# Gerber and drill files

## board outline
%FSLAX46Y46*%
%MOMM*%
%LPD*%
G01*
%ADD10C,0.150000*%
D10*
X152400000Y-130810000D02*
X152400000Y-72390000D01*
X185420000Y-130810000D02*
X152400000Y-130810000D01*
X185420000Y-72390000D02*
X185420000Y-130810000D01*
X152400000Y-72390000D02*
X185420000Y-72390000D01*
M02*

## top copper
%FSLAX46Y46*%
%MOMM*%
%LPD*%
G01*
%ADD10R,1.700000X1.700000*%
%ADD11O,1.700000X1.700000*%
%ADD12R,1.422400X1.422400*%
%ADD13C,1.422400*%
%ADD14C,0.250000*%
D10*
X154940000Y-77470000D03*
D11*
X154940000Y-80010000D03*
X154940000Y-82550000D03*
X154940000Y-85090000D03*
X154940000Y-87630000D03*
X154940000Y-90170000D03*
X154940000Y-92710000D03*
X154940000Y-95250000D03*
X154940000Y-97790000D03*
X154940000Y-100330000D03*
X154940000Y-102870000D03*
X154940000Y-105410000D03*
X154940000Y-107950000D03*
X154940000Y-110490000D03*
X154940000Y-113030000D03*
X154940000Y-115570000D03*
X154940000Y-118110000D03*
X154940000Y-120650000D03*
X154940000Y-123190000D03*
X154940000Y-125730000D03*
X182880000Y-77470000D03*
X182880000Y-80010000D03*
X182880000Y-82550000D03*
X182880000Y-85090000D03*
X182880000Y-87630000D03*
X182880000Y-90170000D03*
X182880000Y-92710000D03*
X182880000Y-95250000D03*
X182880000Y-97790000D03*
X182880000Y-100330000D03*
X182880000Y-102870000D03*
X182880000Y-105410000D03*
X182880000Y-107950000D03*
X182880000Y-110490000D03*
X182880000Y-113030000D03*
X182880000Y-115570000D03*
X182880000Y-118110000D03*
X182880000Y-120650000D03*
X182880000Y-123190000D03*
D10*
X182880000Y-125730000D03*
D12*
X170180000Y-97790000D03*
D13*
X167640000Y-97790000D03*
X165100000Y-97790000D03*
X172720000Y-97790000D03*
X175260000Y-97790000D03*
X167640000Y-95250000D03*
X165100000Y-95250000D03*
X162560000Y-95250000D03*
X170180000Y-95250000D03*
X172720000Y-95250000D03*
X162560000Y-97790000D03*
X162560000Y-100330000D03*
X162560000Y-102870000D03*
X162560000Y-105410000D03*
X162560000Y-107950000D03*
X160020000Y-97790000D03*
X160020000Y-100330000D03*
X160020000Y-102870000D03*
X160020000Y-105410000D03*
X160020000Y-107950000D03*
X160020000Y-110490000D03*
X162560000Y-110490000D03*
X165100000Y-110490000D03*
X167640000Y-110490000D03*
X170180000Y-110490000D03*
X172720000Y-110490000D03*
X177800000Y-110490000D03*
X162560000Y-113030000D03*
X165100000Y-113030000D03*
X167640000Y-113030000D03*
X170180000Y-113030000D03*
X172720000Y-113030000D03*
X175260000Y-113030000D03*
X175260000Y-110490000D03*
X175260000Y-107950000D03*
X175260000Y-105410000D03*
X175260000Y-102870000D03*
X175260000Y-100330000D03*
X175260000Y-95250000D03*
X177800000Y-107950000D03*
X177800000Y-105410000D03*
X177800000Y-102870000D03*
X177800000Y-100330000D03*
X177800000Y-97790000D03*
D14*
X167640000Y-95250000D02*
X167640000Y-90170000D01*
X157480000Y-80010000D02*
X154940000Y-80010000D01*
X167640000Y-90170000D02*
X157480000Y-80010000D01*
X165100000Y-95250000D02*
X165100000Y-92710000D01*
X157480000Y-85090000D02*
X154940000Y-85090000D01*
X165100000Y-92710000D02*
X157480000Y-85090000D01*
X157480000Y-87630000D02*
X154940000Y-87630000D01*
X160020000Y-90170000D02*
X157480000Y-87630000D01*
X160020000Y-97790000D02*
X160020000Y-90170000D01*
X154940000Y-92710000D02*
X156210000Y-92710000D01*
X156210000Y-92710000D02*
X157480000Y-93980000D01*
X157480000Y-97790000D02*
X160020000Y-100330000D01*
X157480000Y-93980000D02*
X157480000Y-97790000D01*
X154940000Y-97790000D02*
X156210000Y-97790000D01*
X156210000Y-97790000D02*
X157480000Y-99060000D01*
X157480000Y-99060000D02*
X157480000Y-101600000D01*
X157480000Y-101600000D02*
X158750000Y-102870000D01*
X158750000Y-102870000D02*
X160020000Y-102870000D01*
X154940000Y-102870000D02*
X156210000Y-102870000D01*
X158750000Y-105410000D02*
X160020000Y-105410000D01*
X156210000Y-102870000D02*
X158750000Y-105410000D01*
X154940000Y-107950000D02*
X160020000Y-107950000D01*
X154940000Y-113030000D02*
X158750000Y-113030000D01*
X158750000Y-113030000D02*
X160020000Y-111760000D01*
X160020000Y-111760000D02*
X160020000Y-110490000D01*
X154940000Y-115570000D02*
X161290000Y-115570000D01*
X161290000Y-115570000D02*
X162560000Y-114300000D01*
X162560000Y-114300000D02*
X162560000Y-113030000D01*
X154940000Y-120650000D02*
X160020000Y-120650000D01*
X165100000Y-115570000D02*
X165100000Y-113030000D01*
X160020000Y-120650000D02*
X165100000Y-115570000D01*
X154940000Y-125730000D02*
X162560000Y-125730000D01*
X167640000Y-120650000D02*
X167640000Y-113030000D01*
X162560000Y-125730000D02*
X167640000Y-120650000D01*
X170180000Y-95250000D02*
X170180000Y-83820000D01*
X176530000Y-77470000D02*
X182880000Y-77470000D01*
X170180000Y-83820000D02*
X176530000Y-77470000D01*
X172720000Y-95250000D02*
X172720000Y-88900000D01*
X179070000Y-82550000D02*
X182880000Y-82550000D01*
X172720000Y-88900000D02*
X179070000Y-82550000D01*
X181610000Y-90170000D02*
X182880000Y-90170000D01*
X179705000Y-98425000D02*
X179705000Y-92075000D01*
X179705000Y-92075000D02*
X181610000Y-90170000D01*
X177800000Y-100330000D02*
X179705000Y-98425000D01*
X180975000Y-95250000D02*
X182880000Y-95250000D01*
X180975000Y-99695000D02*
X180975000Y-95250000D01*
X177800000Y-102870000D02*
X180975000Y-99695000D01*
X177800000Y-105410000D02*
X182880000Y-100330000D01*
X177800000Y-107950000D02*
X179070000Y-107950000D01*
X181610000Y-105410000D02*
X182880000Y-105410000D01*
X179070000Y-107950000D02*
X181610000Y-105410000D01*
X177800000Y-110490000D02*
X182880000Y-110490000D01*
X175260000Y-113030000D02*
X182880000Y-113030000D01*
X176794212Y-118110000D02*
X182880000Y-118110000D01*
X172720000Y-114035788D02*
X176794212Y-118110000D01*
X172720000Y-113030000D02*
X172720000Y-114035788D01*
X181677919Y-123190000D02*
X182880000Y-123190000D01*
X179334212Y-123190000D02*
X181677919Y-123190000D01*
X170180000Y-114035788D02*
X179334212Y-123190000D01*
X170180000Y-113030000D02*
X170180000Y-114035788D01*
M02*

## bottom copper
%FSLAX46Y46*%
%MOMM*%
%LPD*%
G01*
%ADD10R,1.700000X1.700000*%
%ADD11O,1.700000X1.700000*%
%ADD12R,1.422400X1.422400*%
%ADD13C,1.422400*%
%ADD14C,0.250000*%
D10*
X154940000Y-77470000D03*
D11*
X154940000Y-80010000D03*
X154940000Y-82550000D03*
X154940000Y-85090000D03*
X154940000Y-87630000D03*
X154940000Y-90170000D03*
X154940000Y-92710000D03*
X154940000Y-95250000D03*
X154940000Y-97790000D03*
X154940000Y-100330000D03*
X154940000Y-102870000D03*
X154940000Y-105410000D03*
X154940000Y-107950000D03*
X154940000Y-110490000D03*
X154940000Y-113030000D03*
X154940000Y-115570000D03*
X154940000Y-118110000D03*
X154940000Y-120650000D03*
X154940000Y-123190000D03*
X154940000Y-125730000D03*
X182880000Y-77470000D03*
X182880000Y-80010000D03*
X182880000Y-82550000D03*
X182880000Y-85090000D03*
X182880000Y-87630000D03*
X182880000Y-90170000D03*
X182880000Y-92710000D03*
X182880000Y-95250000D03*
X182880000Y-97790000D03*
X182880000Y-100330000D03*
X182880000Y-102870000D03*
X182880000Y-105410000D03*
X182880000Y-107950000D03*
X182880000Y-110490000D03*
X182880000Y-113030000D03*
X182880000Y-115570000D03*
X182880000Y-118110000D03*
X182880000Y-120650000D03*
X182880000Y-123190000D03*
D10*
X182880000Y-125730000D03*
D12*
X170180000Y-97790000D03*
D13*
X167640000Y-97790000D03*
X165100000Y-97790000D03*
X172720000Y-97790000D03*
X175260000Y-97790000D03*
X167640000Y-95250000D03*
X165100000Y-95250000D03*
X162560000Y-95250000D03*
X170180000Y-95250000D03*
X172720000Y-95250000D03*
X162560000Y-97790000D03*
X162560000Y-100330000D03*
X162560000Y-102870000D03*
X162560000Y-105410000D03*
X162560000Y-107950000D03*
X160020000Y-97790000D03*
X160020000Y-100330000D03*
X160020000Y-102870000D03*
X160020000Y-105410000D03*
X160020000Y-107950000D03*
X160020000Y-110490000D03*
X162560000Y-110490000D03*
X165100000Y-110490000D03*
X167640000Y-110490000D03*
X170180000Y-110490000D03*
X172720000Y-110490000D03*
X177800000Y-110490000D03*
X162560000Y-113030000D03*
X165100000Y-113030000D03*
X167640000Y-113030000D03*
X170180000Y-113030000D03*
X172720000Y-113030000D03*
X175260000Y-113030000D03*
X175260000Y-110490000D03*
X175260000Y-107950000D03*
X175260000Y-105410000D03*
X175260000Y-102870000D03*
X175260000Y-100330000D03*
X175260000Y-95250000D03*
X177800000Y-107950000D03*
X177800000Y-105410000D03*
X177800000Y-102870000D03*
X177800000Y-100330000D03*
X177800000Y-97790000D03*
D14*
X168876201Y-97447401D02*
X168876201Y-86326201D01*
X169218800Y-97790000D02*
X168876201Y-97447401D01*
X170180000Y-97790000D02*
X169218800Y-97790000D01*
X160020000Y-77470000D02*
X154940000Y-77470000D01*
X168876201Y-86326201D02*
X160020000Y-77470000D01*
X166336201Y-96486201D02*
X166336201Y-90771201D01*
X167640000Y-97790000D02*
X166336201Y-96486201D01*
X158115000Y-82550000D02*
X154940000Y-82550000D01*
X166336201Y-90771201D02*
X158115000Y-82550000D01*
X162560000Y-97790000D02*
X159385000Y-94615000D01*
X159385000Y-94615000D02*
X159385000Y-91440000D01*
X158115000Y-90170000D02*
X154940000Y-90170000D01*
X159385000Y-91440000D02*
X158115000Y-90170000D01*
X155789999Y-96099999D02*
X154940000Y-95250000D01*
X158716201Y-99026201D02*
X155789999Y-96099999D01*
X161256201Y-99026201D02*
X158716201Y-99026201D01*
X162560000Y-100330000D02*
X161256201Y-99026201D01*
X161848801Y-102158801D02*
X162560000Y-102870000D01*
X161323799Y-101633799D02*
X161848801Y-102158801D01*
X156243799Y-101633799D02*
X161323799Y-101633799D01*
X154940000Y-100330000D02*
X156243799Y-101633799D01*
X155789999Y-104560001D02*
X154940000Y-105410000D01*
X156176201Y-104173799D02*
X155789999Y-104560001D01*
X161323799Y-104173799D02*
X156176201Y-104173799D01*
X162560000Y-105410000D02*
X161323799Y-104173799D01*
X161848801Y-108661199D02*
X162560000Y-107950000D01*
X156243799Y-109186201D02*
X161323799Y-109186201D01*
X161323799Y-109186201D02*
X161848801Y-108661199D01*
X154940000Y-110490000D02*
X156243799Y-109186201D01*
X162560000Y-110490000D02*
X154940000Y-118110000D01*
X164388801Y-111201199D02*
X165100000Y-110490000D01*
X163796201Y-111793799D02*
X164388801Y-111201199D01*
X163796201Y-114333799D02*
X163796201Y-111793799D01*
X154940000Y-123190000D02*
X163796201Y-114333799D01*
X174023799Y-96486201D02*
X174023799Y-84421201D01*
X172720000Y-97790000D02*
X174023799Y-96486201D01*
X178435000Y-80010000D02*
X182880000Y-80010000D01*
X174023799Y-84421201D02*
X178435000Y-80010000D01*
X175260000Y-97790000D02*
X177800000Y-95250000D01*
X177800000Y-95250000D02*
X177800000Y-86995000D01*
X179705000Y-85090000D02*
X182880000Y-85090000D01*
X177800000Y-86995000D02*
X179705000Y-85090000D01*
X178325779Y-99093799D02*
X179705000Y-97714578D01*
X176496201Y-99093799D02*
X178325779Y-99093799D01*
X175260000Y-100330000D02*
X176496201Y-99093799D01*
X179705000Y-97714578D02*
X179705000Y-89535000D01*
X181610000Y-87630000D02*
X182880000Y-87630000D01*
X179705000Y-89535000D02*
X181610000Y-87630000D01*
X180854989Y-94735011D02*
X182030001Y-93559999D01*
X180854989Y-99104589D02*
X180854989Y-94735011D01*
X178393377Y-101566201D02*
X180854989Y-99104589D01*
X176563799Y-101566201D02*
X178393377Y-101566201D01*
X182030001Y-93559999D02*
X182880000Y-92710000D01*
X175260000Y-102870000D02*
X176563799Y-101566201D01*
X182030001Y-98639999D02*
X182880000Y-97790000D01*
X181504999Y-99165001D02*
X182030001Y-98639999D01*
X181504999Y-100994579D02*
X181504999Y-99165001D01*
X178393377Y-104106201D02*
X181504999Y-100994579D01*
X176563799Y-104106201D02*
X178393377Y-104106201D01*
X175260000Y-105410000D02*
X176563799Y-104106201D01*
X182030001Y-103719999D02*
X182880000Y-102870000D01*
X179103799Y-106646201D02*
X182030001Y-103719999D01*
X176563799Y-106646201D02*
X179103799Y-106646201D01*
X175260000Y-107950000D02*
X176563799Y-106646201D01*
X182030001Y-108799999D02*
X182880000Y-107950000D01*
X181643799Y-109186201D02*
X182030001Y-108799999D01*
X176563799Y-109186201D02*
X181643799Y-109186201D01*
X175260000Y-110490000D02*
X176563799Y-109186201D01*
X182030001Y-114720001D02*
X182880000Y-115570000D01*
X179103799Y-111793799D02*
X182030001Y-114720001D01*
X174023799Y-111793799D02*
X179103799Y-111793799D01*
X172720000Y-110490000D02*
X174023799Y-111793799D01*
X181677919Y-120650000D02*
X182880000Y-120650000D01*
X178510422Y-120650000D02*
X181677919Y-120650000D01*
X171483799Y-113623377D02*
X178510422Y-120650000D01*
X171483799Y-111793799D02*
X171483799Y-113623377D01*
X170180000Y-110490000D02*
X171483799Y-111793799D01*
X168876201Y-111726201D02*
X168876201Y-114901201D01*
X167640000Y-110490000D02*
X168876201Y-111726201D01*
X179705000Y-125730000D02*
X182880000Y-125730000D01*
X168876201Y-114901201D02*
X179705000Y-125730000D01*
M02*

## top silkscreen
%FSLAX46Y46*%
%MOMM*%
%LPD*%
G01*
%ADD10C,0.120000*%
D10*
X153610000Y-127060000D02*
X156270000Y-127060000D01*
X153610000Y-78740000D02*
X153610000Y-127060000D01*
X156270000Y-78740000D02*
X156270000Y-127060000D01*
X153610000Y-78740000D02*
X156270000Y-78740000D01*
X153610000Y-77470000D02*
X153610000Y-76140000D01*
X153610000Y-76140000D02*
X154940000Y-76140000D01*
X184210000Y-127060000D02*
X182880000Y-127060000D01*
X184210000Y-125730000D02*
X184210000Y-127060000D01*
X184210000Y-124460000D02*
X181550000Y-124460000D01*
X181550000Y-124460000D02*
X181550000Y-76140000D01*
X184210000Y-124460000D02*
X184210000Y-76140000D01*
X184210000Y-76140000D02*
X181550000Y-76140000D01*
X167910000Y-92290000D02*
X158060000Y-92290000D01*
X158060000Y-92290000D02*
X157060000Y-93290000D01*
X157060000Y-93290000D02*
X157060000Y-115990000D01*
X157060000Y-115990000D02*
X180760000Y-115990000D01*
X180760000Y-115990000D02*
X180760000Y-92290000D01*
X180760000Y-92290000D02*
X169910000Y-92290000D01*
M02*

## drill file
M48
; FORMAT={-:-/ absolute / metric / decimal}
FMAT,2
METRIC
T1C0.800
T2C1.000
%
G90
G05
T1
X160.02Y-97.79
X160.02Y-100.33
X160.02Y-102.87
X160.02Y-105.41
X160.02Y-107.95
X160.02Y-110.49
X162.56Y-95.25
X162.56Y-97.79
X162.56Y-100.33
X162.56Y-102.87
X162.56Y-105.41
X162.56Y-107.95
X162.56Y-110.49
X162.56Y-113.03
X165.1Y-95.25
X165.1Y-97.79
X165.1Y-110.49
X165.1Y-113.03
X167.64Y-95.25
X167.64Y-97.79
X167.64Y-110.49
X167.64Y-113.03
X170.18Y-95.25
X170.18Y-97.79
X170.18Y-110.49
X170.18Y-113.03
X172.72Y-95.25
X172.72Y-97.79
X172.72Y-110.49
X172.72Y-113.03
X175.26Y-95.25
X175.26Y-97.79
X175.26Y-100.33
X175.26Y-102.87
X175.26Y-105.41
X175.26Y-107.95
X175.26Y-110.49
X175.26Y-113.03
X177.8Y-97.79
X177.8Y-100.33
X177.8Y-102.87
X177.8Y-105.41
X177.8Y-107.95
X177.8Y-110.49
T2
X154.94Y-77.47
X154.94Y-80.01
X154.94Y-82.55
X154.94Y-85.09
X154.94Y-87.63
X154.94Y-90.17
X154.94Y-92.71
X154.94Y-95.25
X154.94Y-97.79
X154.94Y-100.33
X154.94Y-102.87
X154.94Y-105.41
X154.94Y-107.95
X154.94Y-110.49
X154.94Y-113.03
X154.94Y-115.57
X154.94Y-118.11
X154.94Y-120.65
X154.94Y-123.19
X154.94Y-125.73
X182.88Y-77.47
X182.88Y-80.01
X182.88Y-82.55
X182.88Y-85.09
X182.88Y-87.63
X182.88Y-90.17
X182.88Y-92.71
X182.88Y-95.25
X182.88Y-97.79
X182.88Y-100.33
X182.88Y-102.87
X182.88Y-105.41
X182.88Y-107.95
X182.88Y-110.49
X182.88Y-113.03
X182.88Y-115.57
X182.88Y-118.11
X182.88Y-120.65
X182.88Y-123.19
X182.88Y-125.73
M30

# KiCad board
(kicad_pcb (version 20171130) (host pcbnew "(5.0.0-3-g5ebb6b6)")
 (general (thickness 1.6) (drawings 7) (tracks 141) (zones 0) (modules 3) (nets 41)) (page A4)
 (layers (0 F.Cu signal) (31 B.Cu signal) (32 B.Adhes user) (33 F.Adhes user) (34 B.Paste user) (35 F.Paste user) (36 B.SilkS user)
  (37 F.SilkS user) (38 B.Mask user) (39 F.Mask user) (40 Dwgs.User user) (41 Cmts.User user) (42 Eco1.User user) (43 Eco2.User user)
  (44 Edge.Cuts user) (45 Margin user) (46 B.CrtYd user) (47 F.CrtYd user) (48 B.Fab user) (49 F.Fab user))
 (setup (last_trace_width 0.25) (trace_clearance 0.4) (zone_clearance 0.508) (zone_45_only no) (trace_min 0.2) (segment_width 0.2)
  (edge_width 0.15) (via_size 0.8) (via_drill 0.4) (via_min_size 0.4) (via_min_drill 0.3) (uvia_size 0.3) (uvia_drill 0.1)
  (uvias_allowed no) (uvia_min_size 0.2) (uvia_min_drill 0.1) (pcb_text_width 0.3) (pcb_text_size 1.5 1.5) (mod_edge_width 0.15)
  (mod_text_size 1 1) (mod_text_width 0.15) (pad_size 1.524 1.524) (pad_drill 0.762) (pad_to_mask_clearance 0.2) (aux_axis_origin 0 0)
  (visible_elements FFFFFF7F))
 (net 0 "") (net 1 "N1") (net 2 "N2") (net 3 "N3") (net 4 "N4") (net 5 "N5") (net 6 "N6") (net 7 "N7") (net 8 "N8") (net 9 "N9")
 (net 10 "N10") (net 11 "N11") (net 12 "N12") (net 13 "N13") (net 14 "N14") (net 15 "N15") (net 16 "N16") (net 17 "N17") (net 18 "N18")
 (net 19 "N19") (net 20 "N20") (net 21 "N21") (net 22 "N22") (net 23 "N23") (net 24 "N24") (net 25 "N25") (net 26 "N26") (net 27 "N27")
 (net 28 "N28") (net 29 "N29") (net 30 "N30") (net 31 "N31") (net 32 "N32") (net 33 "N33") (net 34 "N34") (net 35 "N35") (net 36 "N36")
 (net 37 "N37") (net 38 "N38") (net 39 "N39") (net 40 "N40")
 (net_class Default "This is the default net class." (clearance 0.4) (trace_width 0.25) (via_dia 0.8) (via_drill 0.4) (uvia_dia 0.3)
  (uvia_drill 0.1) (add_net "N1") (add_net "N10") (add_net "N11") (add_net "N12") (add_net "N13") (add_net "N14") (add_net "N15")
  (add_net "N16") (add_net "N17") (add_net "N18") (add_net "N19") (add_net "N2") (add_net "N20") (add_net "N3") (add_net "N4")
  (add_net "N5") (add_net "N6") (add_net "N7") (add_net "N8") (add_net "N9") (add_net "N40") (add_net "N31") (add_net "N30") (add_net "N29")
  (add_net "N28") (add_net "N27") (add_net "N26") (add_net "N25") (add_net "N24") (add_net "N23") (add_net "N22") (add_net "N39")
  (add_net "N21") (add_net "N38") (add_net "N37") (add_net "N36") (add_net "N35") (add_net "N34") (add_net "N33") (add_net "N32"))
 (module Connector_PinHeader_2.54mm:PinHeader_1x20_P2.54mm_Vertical (layer F.Cu) (at 154.94 77.47)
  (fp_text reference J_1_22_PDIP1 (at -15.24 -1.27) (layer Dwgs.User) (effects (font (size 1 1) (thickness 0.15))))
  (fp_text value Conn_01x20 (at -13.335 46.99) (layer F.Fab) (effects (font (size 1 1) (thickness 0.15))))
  (fp_line (start -1.33 49.59) (end 1.33 49.59) (layer F.SilkS) (width 0.12))
  (fp_line (start -1.33 1.27) (end -1.33 49.59) (layer F.SilkS) (width 0.12))
  (fp_line (start 1.33 1.27) (end 1.33 49.59) (layer F.SilkS) (width 0.12))
  (fp_line (start -1.33 1.27) (end 1.33 1.27) (layer F.SilkS) (width 0.12))
  (fp_line (start -1.33 0) (end -1.33 -1.33) (layer F.SilkS) (width 0.12))
  (fp_line (start -1.33 -1.33) (end 0 -1.33) (layer F.SilkS) (width 0.12))
  (pad 1 thru_hole rect (at 0 0) (size 1.7 1.7) (drill 1) (layers *.Cu *.Mask) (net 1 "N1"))
  (pad 2 thru_hole oval (at 0 2.54) (size 1.7 1.7) (drill 1) (layers *.Cu *.Mask) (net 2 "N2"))
  (pad 3 thru_hole oval (at 0 5.08) (size 1.7 1.7) (drill 1) (layers *.Cu *.Mask) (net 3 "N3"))
  (pad 4 thru_hole oval (at 0 7.62) (size 1.7 1.7) (drill 1) (layers *.Cu *.Mask) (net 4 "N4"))
  (pad 5 thru_hole oval (at 0 10.16) (size 1.7 1.7) (drill 1) (layers *.Cu *.Mask) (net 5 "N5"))
  (pad 6 thru_hole oval (at 0 12.7) (size 1.7 1.7) (drill 1) (layers *.Cu *.Mask) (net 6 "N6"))
  (pad 7 thru_hole oval (at 0 15.24) (size 1.7 1.7) (drill 1) (layers *.Cu *.Mask) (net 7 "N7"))
  (pad 8 thru_hole oval (at 0 17.78) (size 1.7 1.7) (drill 1) (layers *.Cu *.Mask) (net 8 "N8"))
  (pad 9 thru_hole oval (at 0 20.32) (size 1.7 1.7) (drill 1) (layers *.Cu *.Mask) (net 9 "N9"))
  (pad 10 thru_hole oval (at 0 22.86) (size 1.7 1.7) (drill 1) (layers *.Cu *.Mask) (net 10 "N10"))
  (pad 11 thru_hole oval (at 0 25.4) (size 1.7 1.7) (drill 1) (layers *.Cu *.Mask) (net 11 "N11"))
  (pad 12 thru_hole oval (at 0 27.94) (size 1.7 1.7) (drill 1) (layers *.Cu *.Mask) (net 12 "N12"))
  (pad 13 thru_hole oval (at 0 30.48) (size 1.7 1.7) (drill 1) (layers *.Cu *.Mask) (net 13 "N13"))
  (pad 14 thru_hole oval (at 0 33.02) (size 1.7 1.7) (drill 1) (layers *.Cu *.Mask) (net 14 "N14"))
  (pad 15 thru_hole oval (at 0 35.56) (size 1.7 1.7) (drill 1) (layers *.Cu *.Mask) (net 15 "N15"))
  (pad 16 thru_hole oval (at 0 38.1) (size 1.7 1.7) (drill 1) (layers *.Cu *.Mask) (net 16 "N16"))
  (pad 17 thru_hole oval (at 0 40.64) (size 1.7 1.7) (drill 1) (layers *.Cu *.Mask) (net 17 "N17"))
  (pad 18 thru_hole oval (at 0 43.18) (size 1.7 1.7) (drill 1) (layers *.Cu *.Mask) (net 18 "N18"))
  (pad 19 thru_hole oval (at 0 45.72) (size 1.7 1.7) (drill 1) (layers *.Cu *.Mask) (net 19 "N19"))
  (pad 20 thru_hole oval (at 0 48.26) (size 1.7 1.7) (drill 1) (layers *.Cu *.Mask) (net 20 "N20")))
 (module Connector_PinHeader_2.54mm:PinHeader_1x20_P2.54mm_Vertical (layer F.Cu) (at 182.88 125.73 180)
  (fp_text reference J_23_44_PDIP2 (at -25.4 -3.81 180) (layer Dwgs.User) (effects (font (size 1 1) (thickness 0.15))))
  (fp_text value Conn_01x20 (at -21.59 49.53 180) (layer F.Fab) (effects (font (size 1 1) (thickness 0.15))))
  (fp_line (start -1.33 -1.33) (end 0 -1.33) (layer F.SilkS) (width 0.12))
  (fp_line (start -1.33 0) (end -1.33 -1.33) (layer F.SilkS) (width 0.12))
  (fp_line (start -1.33 1.27) (end 1.33 1.27) (layer F.SilkS) (width 0.12))
  (fp_line (start 1.33 1.27) (end 1.33 49.59) (layer F.SilkS) (width 0.12))
  (fp_line (start -1.33 1.27) (end -1.33 49.59) (layer F.SilkS) (width 0.12))
  (fp_line (start -1.33 49.59) (end 1.33 49.59) (layer F.SilkS) (width 0.12))
  (pad 20 thru_hole oval (at 0 48.26 180) (size 1.7 1.7) (drill 1) (layers *.Cu *.Mask) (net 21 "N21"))
  (pad 19 thru_hole oval (at 0 45.72 180) (size 1.7 1.7) (drill 1) (layers *.Cu *.Mask) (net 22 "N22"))
  (pad 18 thru_hole oval (at 0 43.18 180) (size 1.7 1.7) (drill 1) (layers *.Cu *.Mask) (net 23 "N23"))
  (pad 17 thru_hole oval (at 0 40.64 180) (size 1.7 1.7) (drill 1) (layers *.Cu *.Mask) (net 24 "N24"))
  (pad 16 thru_hole oval (at 0 38.1 180) (size 1.7 1.7) (drill 1) (layers *.Cu *.Mask) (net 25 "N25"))
  (pad 15 thru_hole oval (at 0 35.56 180) (size 1.7 1.7) (drill 1) (layers *.Cu *.Mask) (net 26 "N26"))
  (pad 14 thru_hole oval (at 0 33.02 180) (size 1.7 1.7) (drill 1) (layers *.Cu *.Mask) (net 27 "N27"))
  (pad 13 thru_hole oval (at 0 30.48 180) (size 1.7 1.7) (drill 1) (layers *.Cu *.Mask) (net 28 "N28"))
  (pad 12 thru_hole oval (at 0 27.94 180) (size 1.7 1.7) (drill 1) (layers *.Cu *.Mask) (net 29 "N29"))
  (pad 11 thru_hole oval (at 0 25.4 180) (size 1.7 1.7) (drill 1) (layers *.Cu *.Mask) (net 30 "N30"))
  (pad 10 thru_hole oval (at 0 22.86 180) (size 1.7 1.7) (drill 1) (layers *.Cu *.Mask) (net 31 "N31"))
  (pad 9 thru_hole oval (at 0 20.32 180) (size 1.7 1.7) (drill 1) (layers *.Cu *.Mask) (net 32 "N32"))
  (pad 8 thru_hole oval (at 0 17.78 180) (size 1.7 1.7) (drill 1) (layers *.Cu *.Mask) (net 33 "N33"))
  (pad 7 thru_hole oval (at 0 15.24 180) (size 1.7 1.7) (drill 1) (layers *.Cu *.Mask) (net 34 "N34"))
  (pad 6 thru_hole oval (at 0 12.7 180) (size 1.7 1.7) (drill 1) (layers *.Cu *.Mask) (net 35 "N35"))
  (pad 5 thru_hole oval (at 0 10.16 180) (size 1.7 1.7) (drill 1) (layers *.Cu *.Mask) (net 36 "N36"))
  (pad 4 thru_hole oval (at 0 7.62 180) (size 1.7 1.7) (drill 1) (layers *.Cu *.Mask) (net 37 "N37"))
  (pad 3 thru_hole oval (at 0 5.08 180) (size 1.7 1.7) (drill 1) (layers *.Cu *.Mask) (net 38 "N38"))
  (pad 2 thru_hole oval (at 0 2.54 180) (size 1.7 1.7) (drill 1) (layers *.Cu *.Mask) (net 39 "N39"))
  (pad 1 thru_hole rect (at 0 0 180) (size 1.7 1.7) (drill 1) (layers *.Cu *.Mask) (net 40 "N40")))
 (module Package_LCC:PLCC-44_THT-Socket (layer F.Cu) (at 170.18 97.79)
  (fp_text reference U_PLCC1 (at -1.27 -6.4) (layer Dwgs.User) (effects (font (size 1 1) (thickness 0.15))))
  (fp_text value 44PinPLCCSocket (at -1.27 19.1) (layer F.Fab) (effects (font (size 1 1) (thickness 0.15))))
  (fp_line (start -2.27 -5.5) (end -12.12 -5.5) (layer F.SilkS) (width 0.12))
  (fp_line (start -12.12 -5.5) (end -13.12 -4.5) (layer F.SilkS) (width 0.12))
  (fp_line (start -13.12 -4.5) (end -13.12 18.2) (layer F.SilkS) (width 0.12))
  (fp_line (start -13.12 18.2) (end 10.58 18.2) (layer F.SilkS) (width 0.12))
  (fp_line (start 10.58 18.2) (end 10.58 -5.5) (layer F.SilkS) (width 0.12))
  (fp_line (start 10.58 -5.5) (end -0.27 -5.5) (layer F.SilkS) (width 0.12))
  (pad 1 thru_hole rect (at 0 0) (size 1.4224 1.4224) (drill 0.8) (layers *.Cu *.Mask) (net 1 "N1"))
  (pad 3 thru_hole circle (at -2.54 0) (size 1.4224 1.4224) (drill 0.8) (layers *.Cu *.Mask) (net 3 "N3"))
  (pad 5 thru_hole circle (at -5.08 0) (size 1.4224 1.4224) (drill 0.8) (layers *.Cu *.Mask))
  (pad 43 thru_hole circle (at 2.54 0) (size 1.4224 1.4224) (drill 0.8) (layers *.Cu *.Mask) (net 22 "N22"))
  (pad 41 thru_hole circle (at 5.08 0) (size 1.4224 1.4224) (drill 0.8) (layers *.Cu *.Mask) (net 24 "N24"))
  (pad 2 thru_hole circle (at -2.54 -2.54) (size 1.4224 1.4224) (drill 0.8) (layers *.Cu *.Mask) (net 2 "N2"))
  (pad 4 thru_hole circle (at -5.08 -2.54) (size 1.4224 1.4224) (drill 0.8) (layers *.Cu *.Mask) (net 4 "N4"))
  (pad 6 thru_hole circle (at -7.62 -2.54) (size 1.4224 1.4224) (drill 0.8) (layers *.Cu *.Mask))
  (pad 44 thru_hole circle (at 0 -2.54) (size 1.4224 1.4224) (drill 0.8) (layers *.Cu *.Mask) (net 21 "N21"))
  (pad 42 thru_hole circle (at 2.54 -2.54) (size 1.4224 1.4224) (drill 0.8) (layers *.Cu *.Mask) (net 23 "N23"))
  (pad 8 thru_hole circle (at -7.62 0) (size 1.4224 1.4224) (drill 0.8) (layers *.Cu *.Mask) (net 6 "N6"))
  (pad 10 thru_hole circle (at -7.62 2.54) (size 1.4224 1.4224) (drill 0.8) (layers *.Cu *.Mask) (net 8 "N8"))
  (pad 12 thru_hole circle (at -7.62 5.08) (size 1.4224 1.4224) (drill 0.8) (layers *.Cu *.Mask) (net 10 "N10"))
  (pad 14 thru_hole circle (at -7.62 7.62) (size 1.4224 1.4224) (drill 0.8) (layers *.Cu *.Mask) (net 12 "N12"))
  (pad 16 thru_hole circle (at -7.62 10.16) (size 1.4224 1.4224) (drill 0.8) (layers *.Cu *.Mask) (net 14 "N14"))
  (pad 7 thru_hole circle (at -10.16 0) (size 1.4224 1.4224) (drill 0.8) (layers *.Cu *.Mask) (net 5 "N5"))
  (pad 9 thru_hole circle (at -10.16 2.54) (size 1.4224 1.4224) (drill 0.8) (layers *.Cu *.Mask) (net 7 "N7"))
  (pad 11 thru_hole circle (at -10.16 5.08) (size 1.4224 1.4224) (drill 0.8) (layers *.Cu *.Mask) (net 9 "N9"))
  (pad 13 thru_hole circle (at -10.16 7.62) (size 1.4224 1.4224) (drill 0.8) (layers *.Cu *.Mask) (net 11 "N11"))
  (pad 15 thru_hole circle (at -10.16 10.16) (size 1.4224 1.4224) (drill 0.8) (layers *.Cu *.Mask) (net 13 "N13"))
  (pad 17 thru_hole circle (at -10.16 12.7) (size 1.4224 1.4224) (drill 0.8) (layers *.Cu *.Mask) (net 15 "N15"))
  (pad 19 thru_hole circle (at -7.62 12.7) (size 1.4224 1.4224) (drill 0.8) (layers *.Cu *.Mask) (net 17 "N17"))
  (pad 21 thru_hole circle (at -5.08 12.7) (size 1.4224 1.4224) (drill 0.8) (layers *.Cu *.Mask) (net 19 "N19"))
  (pad 23 thru_hole circle (at -2.54 12.7) (size 1.4224 1.4224) (drill 0.8) (layers *.Cu *.Mask) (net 40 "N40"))
  (pad 25 thru_hole circle (at 0 12.7) (size 1.4224 1.4224) (drill 0.8) (layers *.Cu *.Mask) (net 38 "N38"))
  (pad 27 thru_hole circle (at 2.54 12.7) (size 1.4224 1.4224) (drill 0.8) (layers *.Cu *.Mask) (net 36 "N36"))
  (pad 29 thru_hole circle (at 7.62 12.7) (size 1.4224 1.4224) (drill 0.8) (layers *.Cu *.Mask) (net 34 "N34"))
  (pad 18 thru_hole circle (at -7.62 15.24) (size 1.4224 1.4224) (drill 0.8) (layers *.Cu *.Mask) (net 16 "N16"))
  (pad 20 thru_hole circle (at -5.08 15.24) (size 1.4224 1.4224) (drill 0.8) (layers *.Cu *.Mask) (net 18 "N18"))
  (pad 22 thru_hole circle (at -2.54 15.24) (size 1.4224 1.4224) (drill 0.8) (layers *.Cu *.Mask) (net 20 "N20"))
  (pad 24 thru_hole circle (at 0 15.24) (size 1.4224 1.4224) (drill 0.8) (layers *.Cu *.Mask) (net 39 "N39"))
  (pad 26 thru_hole circle (at 2.54 15.24) (size 1.4224 1.4224) (drill 0.8) (layers *.Cu *.Mask) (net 37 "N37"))
  (pad 28 thru_hole circle (at 5.08 15.24) (size 1.4224 1.4224) (drill 0.8) (layers *.Cu *.Mask) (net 35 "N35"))
  (pad 30 thru_hole circle (at 5.08 12.7) (size 1.4224 1.4224) (drill 0.8) (layers *.Cu *.Mask) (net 33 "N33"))
  (pad 32 thru_hole circle (at 5.08 10.16) (size 1.4224 1.4224) (drill 0.8) (layers *.Cu *.Mask) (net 31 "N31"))
  (pad 34 thru_hole circle (at 5.08 7.62) (size 1.4224 1.4224) (drill 0.8) (layers *.Cu *.Mask) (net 29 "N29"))
  (pad 36 thru_hole circle (at 5.08 5.08) (size 1.4224 1.4224) (drill 0.8) (layers *.Cu *.Mask) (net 27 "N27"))
  (pad 38 thru_hole circle (at 5.08 2.54) (size 1.4224 1.4224) (drill 0.8) (layers *.Cu *.Mask) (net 25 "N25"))
  (pad 40 thru_hole circle (at 5.08 -2.54) (size 1.4224 1.4224) (drill 0.8) (layers *.Cu *.Mask))
  (pad 31 thru_hole circle (at 7.62 10.16) (size 1.4224 1.4224) (drill 0.8) (layers *.Cu *.Mask) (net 32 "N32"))
  (pad 33 thru_hole circle (at 7.62 7.62) (size 1.4224 1.4224) (drill 0.8) (layers *.Cu *.Mask) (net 30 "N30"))
  (pad 35 thru_hole circle (at 7.62 5.08) (size 1.4224 1.4224) (drill 0.8) (layers *.Cu *.Mask) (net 28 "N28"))
  (pad 37 thru_hole circle (at 7.62 2.54) (size 1.4224 1.4224) (drill 0.8) (layers *.Cu *.Mask) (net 26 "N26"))
  (pad 39 thru_hole circle (at 7.62 0) (size 1.4224 1.4224) (drill 0.8) (layers *.Cu *.Mask)))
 (gr_line (start 152.4 130.81) (end 152.4 72.39) (layer Edge.Cuts) (width 0.15))
 (gr_line (start 185.42 130.81) (end 152.4 130.81) (layer Edge.Cuts) (width 0.15))
 (gr_line (start 185.42 72.39) (end 185.42 130.81) (layer Edge.Cuts) (width 0.15))
 (gr_line (start 152.4 72.39) (end 185.42 72.39) (layer Edge.Cuts) (width 0.15))
 (segment (start 168.876201 97.447401) (end 168.876201 86.326201) (width 0.25) (layer B.Cu) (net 1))
 (segment (start 169.2188 97.79) (end 168.876201 97.447401) (width 0.25) (layer B.Cu) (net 1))
 (segment (start 170.18 97.79) (end 169.2188 97.79) (width 0.25) (layer B.Cu) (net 1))
 (segment (start 160.02 77.47) (end 154.94 77.47) (width 0.25) (layer B.Cu) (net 1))
 (segment (start 168.876201 86.326201) (end 160.02 77.47) (width 0.25) (layer B.Cu) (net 1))
 (segment (start 167.64 95.25) (end 167.64 90.17) (width 0.25) (layer F.Cu) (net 2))
 (segment (start 157.48 80.01) (end 154.94 80.01) (width 0.25) (layer F.Cu) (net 2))
 (segment (start 167.64 90.17) (end 157.48 80.01) (width 0.25) (layer F.Cu) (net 2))
 (segment (start 166.336201 96.486201) (end 166.336201 90.771201) (width 0.25) (layer B.Cu) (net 3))
 (segment (start 167.64 97.79) (end 166.336201 96.486201) (width 0.25) (layer B.Cu) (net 3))
 (segment (start 158.115 82.55) (end 154.94 82.55) (width 0.25) (layer B.Cu) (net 3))
 (segment (start 166.336201 90.771201) (end 158.115 82.55) (width 0.25) (layer B.Cu) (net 3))
 (segment (start 165.1 95.25) (end 165.1 92.71) (width 0.25) (layer F.Cu) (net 4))
 (segment (start 157.48 85.09) (end 154.94 85.09) (width 0.25) (layer F.Cu) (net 4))
 (segment (start 165.1 92.71) (end 157.48 85.09) (width 0.25) (layer F.Cu) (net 4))
 (segment (start 157.48 87.63) (end 154.94 87.63) (width 0.25) (layer F.Cu) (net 5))
 (segment (start 160.02 90.17) (end 157.48 87.63) (width 0.25) (layer F.Cu) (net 5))
 (segment (start 160.02 97.79) (end 160.02 90.17) (width 0.25) (layer F.Cu) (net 5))
 (segment (start 162.56 97.79) (end 159.385 94.615) (width 0.25) (layer B.Cu) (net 6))
 (segment (start 159.385 94.615) (end 159.385 91.44) (width 0.25) (layer B.Cu) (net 6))
 (segment (start 158.115 90.17) (end 154.94 90.17) (width 0.25) (layer B.Cu) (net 6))
 (segment (start 159.385 91.44) (end 158.115 90.17) (width 0.25) (layer B.Cu) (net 6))
 (segment (start 154.94 92.71) (end 156.21 92.71) (width 0.25) (layer F.Cu) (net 7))
 (segment (start 156.21 92.71) (end 157.48 93.98) (width 0.25) (layer F.Cu) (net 7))
 (segment (start 157.48 97.79) (end 160.02 100.33) (width 0.25) (layer F.Cu) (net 7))
 (segment (start 157.48 93.98) (end 157.48 97.79) (width 0.25) (layer F.Cu) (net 7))
 (segment (start 155.789999 96.099999) (end 154.94 95.25) (width 0.25) (layer B.Cu) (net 8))
 (segment (start 158.716201 99.026201) (end 155.789999 96.099999) (width 0.25) (layer B.Cu) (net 8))
 (segment (start 161.256201 99.026201) (end 158.716201 99.026201) (width 0.25) (layer B.Cu) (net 8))
 (segment (start 162.56 100.33) (end 161.256201 99.026201) (width 0.25) (layer B.Cu) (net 8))
 (segment (start 154.94 97.79) (end 156.21 97.79) (width 0.25) (layer F.Cu) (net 9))
 (segment (start 156.21 97.79) (end 157.48 99.06) (width 0.25) (layer F.Cu) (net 9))
 (segment (start 157.48 99.06) (end 157.48 101.6) (width 0.25) (layer F.Cu) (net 9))
 (segment (start 157.48 101.6) (end 158.75 102.87) (width 0.25) (layer F.Cu) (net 9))
 (segment (start 158.75 102.87) (end 160.02 102.87) (width 0.25) (layer F.Cu) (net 9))
 (segment (start 161.848801 102.158801) (end 162.56 102.87) (width 0.25) (layer B.Cu) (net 10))
 (segment (start 161.323799 101.633799) (end 161.848801 102.158801) (width 0.25) (layer B.Cu) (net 10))
 (segment (start 156.243799 101.633799) (end 161.323799 101.633799) (width 0.25) (layer B.Cu) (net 10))
 (segment (start 154.94 100.33) (end 156.243799 101.633799) (width 0.25) (layer B.Cu) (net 10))
 (segment (start 154.94 102.87) (end 156.21 102.87) (width 0.25) (layer F.Cu) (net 11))
 (segment (start 158.75 105.41) (end 160.02 105.41) (width 0.25) (layer F.Cu) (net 11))
 (segment (start 156.21 102.87) (end 158.75 105.41) (width 0.25) (layer F.Cu) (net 11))
 (segment (start 155.789999 104.560001) (end 154.94 105.41) (width 0.25) (layer B.Cu) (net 12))
 (segment (start 156.176201 104.173799) (end 155.789999 104.560001) (width 0.25) (layer B.Cu) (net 12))
 (segment (start 161.323799 104.173799) (end 156.176201 104.173799) (width 0.25) (layer B.Cu) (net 12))
 (segment (start 162.56 105.41) (end 161.323799 104.173799) (width 0.25) (layer B.Cu) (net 12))
 (segment (start 154.94 107.95) (end 160.02 107.95) (width 0.25) (layer F.Cu) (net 13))
 (segment (start 161.848801 108.661199) (end 162.56 107.95) (width 0.25) (layer B.Cu) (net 14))
 (segment (start 156.243799 109.186201) (end 161.323799 109.186201) (width 0.25) (layer B.Cu) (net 14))
 (segment (start 161.323799 109.186201) (end 161.848801 108.661199) (width 0.25) (layer B.Cu) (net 14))
 (segment (start 154.94 110.49) (end 156.243799 109.186201) (width 0.25) (layer B.Cu) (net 14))
 (segment (start 154.94 113.03) (end 158.75 113.03) (width 0.25) (layer F.Cu) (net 15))
 (segment (start 158.75 113.03) (end 160.02 111.76) (width 0.25) (layer F.Cu) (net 15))
 (segment (start 160.02 111.76) (end 160.02 110.49) (width 0.25) (layer F.Cu) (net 15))
 (segment (start 154.94 115.57) (end 161.29 115.57) (width 0.25) (layer F.Cu) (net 16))
 (segment (start 161.29 115.57) (end 162.56 114.3) (width 0.25) (layer F.Cu) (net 16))
 (segment (start 162.56 114.3) (end 162.56 113.03) (width 0.25) (layer F.Cu) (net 16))
 (segment (start 162.56 110.49) (end 154.94 118.11) (width 0.25) (layer B.Cu) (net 17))
 (segment (start 154.94 120.65) (end 160.02 120.65) (width 0.25) (layer F.Cu) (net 18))
 (segment (start 165.1 115.57) (end 165.1 113.03) (width 0.25) (layer F.Cu) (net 18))
 (segment (start 160.02 120.65) (end 165.1 115.57) (width 0.25) (layer F.Cu) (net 18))
 (segment (start 164.388801 111.201199) (end 165.1 110.49) (width 0.25) (layer B.Cu) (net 19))
 (segment (start 163.796201 111.793799) (end 164.388801 111.201199) (width 0.25) (layer B.Cu) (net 19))
 (segment (start 163.796201 114.333799) (end 163.796201 111.793799) (width 0.25) (layer B.Cu) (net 19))
 (segment (start 154.94 123.19) (end 163.796201 114.333799) (width 0.25) (layer B.Cu) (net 19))
 (segment (start 154.94 125.73) (end 162.56 125.73) (width 0.25) (layer F.Cu) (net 20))
 (segment (start 167.64 120.65) (end 167.64 113.03) (width 0.25) (layer F.Cu) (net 20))
 (segment (start 162.56 125.73) (end 167.64 120.65) (width 0.25) (layer F.Cu) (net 20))
 (segment (start 170.18 95.25) (end 170.18 83.82) (width 0.25) (layer F.Cu) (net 21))
 (segment (start 176.53 77.47) (end 182.88 77.47) (width 0.25) (layer F.Cu) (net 21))
 (segment (start 170.18 83.82) (end 176.53 77.47) (width 0.25) (layer F.Cu) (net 21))
 (segment (start 174.023799 96.486201) (end 174.023799 84.421201) (width 0.25) (layer B.Cu) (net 22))
 (segment (start 172.72 97.79) (end 174.023799 96.486201) (width 0.25) (layer B.Cu) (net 22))
 (segment (start 178.435 80.01) (end 182.88 80.01) (width 0.25) (layer B.Cu) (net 22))
 (segment (start 174.023799 84.421201) (end 178.435 80.01) (width 0.25) (layer B.Cu) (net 22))
 (segment (start 172.72 95.25) (end 172.72 88.9) (width 0.25) (layer F.Cu) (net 23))
 (segment (start 179.07 82.55) (end 182.88 82.55) (width 0.25) (layer F.Cu) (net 23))
 (segment (start 172.72 88.9) (end 179.07 82.55) (width 0.25) (layer F.Cu) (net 23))
 (segment (start 175.26 97.79) (end 177.8 95.25) (width 0.25) (layer B.Cu) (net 24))
 (segment (start 177.8 95.25) (end 177.8 86.995) (width 0.25) (layer B.Cu) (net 24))
 (segment (start 179.705 85.09) (end 182.88 85.09) (width 0.25) (layer B.Cu) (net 24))
 (segment (start 177.8 86.995) (end 179.705 85.09) (width 0.25) (layer B.Cu) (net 24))
 (segment (start 178.325779 99.093799) (end 179.705 97.714578) (width 0.25) (layer B.Cu) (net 25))
 (segment (start 176.496201 99.093799) (end 178.325779 99.093799) (width 0.25) (layer B.Cu) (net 25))
 (segment (start 175.26 100.33) (end 176.496201 99.093799) (width 0.25) (layer B.Cu) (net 25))
 (segment (start 179.705 97.714578) (end 179.705 89.535) (width 0.25) (layer B.Cu) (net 25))
 (segment (start 181.61 87.63) (end 182.88 87.63) (width 0.25) (layer B.Cu) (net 25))
 (segment (start 179.705 89.535) (end 181.61 87.63) (width 0.25) (layer B.Cu) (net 25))
 (segment (start 181.61 90.17) (end 182.88 90.17) (width 0.25) (layer F.Cu) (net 26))
 (segment (start 179.705 98.425) (end 179.705 92.075) (width 0.25) (layer F.Cu) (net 26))
 (segment (start 179.705 92.075) (end 181.61 90.17) (width 0.25) (layer F.Cu) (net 26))
 (segment (start 177.8 100.33) (end 179.705 98.425) (width 0.25) (layer F.Cu) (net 26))
 (segment (start 180.854989 94.735011) (end 182.030001 93.559999) (width 0.25) (layer B.Cu) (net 27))
 (segment (start 180.854989 99.104589) (end 180.854989 94.735011) (width 0.25) (layer B.Cu) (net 27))
 (segment (start 178.393377 101.566201) (end 180.854989 99.104589) (width 0.25) (layer B.Cu) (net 27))
 (segment (start 176.563799 101.566201) (end 178.393377 101.566201) (width 0.25) (layer B.Cu) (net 27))
 (segment (start 182.030001 93.559999) (end 182.88 92.71) (width 0.25) (layer B.Cu) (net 27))
 (segment (start 175.26 102.87) (end 176.563799 101.566201) (width 0.25) (layer B.Cu) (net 27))
 (segment (start 180.975 95.25) (end 182.88 95.25) (width 0.25) (layer F.Cu) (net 28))
 (segment (start 180.975 99.695) (end 180.975 95.25) (width 0.25) (layer F.Cu) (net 28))
 (segment (start 177.8 102.87) (end 180.975 99.695) (width 0.25) (layer F.Cu) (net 28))
 (segment (start 182.030001 98.639999) (end 182.88 97.79) (width 0.25) (layer B.Cu) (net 29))
 (segment (start 181.504999 99.165001) (end 182.030001 98.639999) (width 0.25) (layer B.Cu) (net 29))
 (segment (start 181.504999 100.994579) (end 181.504999 99.165001) (width 0.25) (layer B.Cu) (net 29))
 (segment (start 178.393377 104.106201) (end 181.504999 100.994579) (width 0.25) (layer B.Cu) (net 29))
 (segment (start 176.563799 104.106201) (end 178.393377 104.106201) (width 0.25) (layer B.Cu) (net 29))
 (segment (start 175.26 105.41) (end 176.563799 104.106201) (width 0.25) (layer B.Cu) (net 29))
 (segment (start 177.8 105.41) (end 182.88 100.33) (width 0.25) (layer F.Cu) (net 30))
 (segment (start 182.030001 103.719999) (end 182.88 102.87) (width 0.25) (layer B.Cu) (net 31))
 (segment (start 179.103799 106.646201) (end 182.030001 103.719999) (width 0.25) (layer B.Cu) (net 31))
 (segment (start 176.563799 106.646201) (end 179.103799 106.646201) (width 0.25) (layer B.Cu) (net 31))
 (segment (start 175.26 107.95) (end 176.563799 106.646201) (width 0.25) (layer B.Cu) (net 31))
 (segment (start 177.8 107.95) (end 179.07 107.95) (width 0.25) (layer F.Cu) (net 32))
 (segment (start 181.61 105.41) (end 182.88 105.41) (width 0.25) (layer F.Cu) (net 32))
 (segment (start 179.07 107.95) (end 181.61 105.41) (width 0.25) (layer F.Cu) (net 32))
 (segment (start 182.030001 108.799999) (end 182.88 107.95) (width 0.25) (layer B.Cu) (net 33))
 (segment (start 181.643799 109.186201) (end 182.030001 108.799999) (width 0.25) (layer B.Cu) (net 33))
 (segment (start 176.563799 109.186201) (end 181.643799 109.186201) (width 0.25) (layer B.Cu) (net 33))
 (segment (start 175.26 110.49) (end 176.563799 109.186201) (width 0.25) (layer B.Cu) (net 33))
 (segment (start 177.8 110.49) (end 182.88 110.49) (width 0.25) (layer F.Cu) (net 34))
 (segment (start 175.26 113.03) (end 182.88 113.03) (width 0.25) (layer F.Cu) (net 35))
 (segment (start 182.030001 114.720001) (end 182.88 115.57) (width 0.25) (layer B.Cu) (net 36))
 (segment (start 179.103799 111.793799) (end 182.030001 114.720001) (width 0.25) (layer B.Cu) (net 36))
 (segment (start 174.023799 111.793799) (end 179.103799 111.793799) (width 0.25) (layer B.Cu) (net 36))
 (segment (start 172.72 110.49) (end 174.023799 111.793799) (width 0.25) (layer B.Cu) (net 36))
 (segment (start 176.794212 118.11) (end 182.88 118.11) (width 0.25) (layer F.Cu) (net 37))
 (segment (start 172.72 114.035788) (end 176.794212 118.11) (width 0.25) (layer F.Cu) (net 37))
 (segment (start 172.72 113.03) (end 172.72 114.035788) (width 0.25) (layer F.Cu) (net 37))
 (segment (start 181.677919 120.65) (end 182.88 120.65) (width 0.25) (layer B.Cu) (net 38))
 (segment (start 178.510422 120.65) (end 181.677919 120.65) (width 0.25) (layer B.Cu) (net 38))
 (segment (start 171.483799 113.623377) (end 178.510422 120.65) (width 0.25) (layer B.Cu) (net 38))
 (segment (start 171.483799 111.793799) (end 171.483799 113.623377) (width 0.25) (layer B.Cu) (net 38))
 (segment (start 170.18 110.49) (end 171.483799 111.793799) (width 0.25) (layer B.Cu) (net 38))
 (segment (start 181.677919 123.19) (end 182.88 123.19) (width 0.25) (layer F.Cu) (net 39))
 (segment (start 179.334212 123.19) (end 181.677919 123.19) (width 0.25) (layer F.Cu) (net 39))
 (segment (start 170.18 114.035788) (end 179.334212 123.19) (width 0.25) (layer F.Cu) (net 39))
 (segment (start 170.18 113.03) (end 170.18 114.035788) (width 0.25) (layer F.Cu) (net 39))
 (segment (start 168.876201 111.726201) (end 168.876201 114.901201) (width 0.25) (layer B.Cu) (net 40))
 (segment (start 167.64 110.49) (end 168.876201 111.726201) (width 0.25) (layer B.Cu) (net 40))
 (segment (start 179.705 125.73) (end 182.88 125.73) (width 0.25) (layer B.Cu) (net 40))
 (segment (start 168.876201 114.901201) (end 179.705 125.73) (width 0.25) (layer B.Cu) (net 40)))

